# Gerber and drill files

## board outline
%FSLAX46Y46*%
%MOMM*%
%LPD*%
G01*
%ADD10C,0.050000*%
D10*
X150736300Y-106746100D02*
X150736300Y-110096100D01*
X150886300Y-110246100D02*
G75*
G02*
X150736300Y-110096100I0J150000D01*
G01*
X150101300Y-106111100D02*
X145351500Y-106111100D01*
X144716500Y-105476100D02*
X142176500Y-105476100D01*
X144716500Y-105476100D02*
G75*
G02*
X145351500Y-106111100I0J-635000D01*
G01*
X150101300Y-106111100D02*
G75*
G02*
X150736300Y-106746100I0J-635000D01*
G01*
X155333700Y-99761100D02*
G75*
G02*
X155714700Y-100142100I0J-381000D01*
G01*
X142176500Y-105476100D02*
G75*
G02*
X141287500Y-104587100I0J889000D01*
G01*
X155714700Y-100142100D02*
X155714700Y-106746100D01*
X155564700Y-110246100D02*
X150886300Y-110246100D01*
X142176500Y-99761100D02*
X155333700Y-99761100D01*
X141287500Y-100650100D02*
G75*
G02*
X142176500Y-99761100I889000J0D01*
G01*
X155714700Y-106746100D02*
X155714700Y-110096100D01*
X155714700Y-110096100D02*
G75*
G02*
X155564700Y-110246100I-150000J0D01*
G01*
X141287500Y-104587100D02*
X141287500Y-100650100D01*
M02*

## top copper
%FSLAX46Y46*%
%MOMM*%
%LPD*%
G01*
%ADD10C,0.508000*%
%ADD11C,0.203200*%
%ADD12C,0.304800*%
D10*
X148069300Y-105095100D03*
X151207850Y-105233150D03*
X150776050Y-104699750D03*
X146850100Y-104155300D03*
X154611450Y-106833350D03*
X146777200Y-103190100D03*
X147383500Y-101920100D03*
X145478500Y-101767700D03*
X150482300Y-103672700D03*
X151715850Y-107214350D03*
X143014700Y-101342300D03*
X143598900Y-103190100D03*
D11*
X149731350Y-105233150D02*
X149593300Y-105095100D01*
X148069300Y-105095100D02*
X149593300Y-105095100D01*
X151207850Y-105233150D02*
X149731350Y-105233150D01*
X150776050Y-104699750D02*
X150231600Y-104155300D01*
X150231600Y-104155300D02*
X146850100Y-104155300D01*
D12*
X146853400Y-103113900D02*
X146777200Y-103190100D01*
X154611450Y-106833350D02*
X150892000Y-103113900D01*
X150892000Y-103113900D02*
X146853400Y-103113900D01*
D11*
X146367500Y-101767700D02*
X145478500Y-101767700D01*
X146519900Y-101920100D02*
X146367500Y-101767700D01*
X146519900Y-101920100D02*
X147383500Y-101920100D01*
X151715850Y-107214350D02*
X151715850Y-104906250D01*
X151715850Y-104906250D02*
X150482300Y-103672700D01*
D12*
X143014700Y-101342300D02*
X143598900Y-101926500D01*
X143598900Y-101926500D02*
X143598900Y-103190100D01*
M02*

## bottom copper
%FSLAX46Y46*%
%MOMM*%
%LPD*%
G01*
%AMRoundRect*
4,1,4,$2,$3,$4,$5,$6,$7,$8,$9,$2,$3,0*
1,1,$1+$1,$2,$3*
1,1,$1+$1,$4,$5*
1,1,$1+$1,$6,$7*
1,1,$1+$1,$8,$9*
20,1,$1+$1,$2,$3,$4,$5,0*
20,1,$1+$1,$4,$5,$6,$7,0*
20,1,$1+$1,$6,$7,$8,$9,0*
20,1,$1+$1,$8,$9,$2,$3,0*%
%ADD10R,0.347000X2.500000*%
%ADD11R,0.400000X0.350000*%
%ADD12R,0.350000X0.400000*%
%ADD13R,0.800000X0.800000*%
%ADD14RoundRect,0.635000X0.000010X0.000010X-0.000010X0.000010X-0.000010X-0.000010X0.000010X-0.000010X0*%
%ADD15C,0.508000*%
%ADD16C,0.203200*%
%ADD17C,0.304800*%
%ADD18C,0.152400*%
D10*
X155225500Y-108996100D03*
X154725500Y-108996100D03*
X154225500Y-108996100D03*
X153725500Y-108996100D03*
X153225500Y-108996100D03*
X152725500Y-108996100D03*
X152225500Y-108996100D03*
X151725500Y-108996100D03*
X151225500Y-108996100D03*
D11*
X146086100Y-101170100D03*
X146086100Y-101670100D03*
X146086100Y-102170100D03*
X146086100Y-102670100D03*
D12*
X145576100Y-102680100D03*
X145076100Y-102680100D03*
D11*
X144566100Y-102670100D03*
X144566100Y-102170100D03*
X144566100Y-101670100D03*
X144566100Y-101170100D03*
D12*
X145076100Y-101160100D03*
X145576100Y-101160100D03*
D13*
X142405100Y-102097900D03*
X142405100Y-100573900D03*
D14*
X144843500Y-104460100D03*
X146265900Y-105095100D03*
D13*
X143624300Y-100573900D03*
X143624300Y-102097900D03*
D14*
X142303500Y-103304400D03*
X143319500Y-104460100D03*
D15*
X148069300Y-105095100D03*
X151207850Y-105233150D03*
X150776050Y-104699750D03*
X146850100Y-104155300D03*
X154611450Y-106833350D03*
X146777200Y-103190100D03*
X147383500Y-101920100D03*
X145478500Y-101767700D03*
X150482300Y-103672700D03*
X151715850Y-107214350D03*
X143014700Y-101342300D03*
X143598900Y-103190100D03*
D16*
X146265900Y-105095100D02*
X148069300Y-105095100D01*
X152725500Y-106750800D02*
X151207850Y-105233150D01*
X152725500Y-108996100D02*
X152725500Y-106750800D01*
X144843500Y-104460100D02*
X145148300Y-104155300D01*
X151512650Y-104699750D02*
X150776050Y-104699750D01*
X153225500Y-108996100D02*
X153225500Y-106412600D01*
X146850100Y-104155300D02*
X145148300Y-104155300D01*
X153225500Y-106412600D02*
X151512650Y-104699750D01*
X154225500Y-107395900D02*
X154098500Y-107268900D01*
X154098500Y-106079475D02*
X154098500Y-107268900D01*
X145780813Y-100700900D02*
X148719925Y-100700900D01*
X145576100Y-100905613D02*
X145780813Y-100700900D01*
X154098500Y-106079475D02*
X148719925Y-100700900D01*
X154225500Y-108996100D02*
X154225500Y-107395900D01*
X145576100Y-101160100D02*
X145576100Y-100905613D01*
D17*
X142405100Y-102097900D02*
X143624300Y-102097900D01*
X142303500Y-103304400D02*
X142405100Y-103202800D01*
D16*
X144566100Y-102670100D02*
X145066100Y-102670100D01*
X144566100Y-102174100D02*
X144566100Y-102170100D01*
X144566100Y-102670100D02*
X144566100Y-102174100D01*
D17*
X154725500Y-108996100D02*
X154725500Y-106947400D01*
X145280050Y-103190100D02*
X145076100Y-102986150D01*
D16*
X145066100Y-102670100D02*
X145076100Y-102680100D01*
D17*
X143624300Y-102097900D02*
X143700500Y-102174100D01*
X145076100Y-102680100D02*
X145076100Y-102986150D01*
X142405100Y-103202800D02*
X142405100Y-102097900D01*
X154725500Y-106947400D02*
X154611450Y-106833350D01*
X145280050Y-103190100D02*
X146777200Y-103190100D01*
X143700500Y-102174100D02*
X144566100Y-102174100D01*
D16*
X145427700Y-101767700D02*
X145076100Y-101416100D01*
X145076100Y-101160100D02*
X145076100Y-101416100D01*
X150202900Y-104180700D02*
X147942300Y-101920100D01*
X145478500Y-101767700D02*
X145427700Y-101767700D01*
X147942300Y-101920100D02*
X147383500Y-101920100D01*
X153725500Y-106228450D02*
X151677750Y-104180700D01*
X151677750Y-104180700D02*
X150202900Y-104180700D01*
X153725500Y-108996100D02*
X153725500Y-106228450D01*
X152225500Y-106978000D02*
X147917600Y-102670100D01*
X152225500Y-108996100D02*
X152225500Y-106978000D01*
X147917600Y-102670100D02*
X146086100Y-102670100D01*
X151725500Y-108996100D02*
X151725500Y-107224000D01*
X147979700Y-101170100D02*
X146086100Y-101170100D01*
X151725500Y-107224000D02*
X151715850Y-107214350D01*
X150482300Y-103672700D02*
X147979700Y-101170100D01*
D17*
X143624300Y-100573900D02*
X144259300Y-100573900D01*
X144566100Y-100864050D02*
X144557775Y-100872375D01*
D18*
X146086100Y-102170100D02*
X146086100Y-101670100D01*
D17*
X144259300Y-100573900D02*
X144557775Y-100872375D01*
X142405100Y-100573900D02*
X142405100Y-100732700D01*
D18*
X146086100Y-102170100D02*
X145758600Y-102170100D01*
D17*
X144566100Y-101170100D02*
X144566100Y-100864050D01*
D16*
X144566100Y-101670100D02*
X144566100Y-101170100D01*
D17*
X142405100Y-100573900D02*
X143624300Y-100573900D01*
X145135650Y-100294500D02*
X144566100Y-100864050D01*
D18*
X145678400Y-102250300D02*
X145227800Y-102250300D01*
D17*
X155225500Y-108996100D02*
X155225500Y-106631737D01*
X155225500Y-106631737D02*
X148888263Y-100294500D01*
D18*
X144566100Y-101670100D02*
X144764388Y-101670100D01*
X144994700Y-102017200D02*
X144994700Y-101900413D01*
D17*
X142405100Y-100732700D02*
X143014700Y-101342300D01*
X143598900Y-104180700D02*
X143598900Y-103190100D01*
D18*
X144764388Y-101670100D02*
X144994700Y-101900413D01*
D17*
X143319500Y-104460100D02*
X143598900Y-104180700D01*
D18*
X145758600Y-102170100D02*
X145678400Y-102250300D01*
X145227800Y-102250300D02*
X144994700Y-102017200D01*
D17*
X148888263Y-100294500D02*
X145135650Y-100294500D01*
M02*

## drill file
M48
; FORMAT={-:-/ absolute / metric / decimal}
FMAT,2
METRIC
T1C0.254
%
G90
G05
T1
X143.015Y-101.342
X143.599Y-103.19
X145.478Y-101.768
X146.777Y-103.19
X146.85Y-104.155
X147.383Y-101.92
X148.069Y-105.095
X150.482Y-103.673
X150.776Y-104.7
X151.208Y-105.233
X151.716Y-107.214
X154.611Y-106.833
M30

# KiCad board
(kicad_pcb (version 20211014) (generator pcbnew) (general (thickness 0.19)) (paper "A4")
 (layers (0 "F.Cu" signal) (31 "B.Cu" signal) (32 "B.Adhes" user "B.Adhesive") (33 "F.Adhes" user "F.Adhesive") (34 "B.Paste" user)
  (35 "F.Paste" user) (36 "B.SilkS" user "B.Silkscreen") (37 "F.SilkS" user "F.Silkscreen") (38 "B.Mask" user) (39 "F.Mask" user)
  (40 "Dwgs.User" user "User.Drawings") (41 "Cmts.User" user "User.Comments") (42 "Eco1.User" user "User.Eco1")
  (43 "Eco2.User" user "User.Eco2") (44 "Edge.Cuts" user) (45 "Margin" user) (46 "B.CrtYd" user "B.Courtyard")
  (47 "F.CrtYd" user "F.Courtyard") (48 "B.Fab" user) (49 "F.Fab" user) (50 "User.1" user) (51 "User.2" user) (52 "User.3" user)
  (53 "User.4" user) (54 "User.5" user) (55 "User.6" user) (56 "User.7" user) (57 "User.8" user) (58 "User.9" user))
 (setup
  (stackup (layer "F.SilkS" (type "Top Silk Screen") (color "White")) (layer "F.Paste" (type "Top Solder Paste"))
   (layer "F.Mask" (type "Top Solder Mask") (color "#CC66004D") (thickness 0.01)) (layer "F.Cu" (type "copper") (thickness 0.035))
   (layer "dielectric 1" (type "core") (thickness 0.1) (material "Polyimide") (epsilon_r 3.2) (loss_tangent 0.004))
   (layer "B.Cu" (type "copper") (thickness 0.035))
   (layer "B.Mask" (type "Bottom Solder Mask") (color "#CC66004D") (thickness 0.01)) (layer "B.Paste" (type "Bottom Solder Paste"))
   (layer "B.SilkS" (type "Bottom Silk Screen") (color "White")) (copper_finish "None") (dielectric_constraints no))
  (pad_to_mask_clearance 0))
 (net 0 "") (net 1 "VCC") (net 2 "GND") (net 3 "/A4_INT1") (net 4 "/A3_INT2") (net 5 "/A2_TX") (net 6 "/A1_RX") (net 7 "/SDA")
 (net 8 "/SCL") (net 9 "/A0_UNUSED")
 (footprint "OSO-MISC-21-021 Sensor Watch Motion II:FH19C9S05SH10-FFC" (layer "F.Cu") (at 153.2255 106.7461)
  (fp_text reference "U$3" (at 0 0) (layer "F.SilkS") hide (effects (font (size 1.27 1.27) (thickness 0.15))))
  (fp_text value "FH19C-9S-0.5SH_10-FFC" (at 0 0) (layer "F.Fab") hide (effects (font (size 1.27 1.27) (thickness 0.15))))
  (pad "1" smd rect (at 2 2.25 90) (size 2.5 0.347) (layers "B.Cu" "B.Mask") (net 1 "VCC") (solder_mask_margin 0.0635))
  (pad "2" smd rect (at 1.5 2.25 90) (size 2.5 0.347) (layers "B.Cu" "B.Mask") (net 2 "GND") (solder_mask_margin 0.0635))
  (pad "3" smd rect (at 1 2.25 90) (size 2.5 0.347) (layers "B.Cu" "B.Mask") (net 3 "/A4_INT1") (solder_mask_margin 0.0635))
  (pad "4" smd rect (at 0.5 2.25 90) (size 2.5 0.347) (layers "B.Cu" "B.Mask") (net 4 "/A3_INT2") (solder_mask_margin 0.0635))
  (pad "5" smd rect (at 0 2.25 90) (size 2.5 0.347) (layers "B.Cu" "B.Mask") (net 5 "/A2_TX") (solder_mask_margin 0.0635))
  (pad "6" smd rect (at -0.5 2.25 90) (size 2.5 0.347) (layers "B.Cu" "B.Mask") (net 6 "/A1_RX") (solder_mask_margin 0.0635))
  (pad "7" smd rect (at -1 2.25 90) (size 2.5 0.347) (layers "B.Cu" "B.Mask") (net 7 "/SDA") (solder_mask_margin 0.0635))
  (pad "8" smd rect (at -1.5 2.25 90) (size 2.5 0.347) (layers "B.Cu" "B.Mask") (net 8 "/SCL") (solder_mask_margin 0.0635))
  (pad "9" smd rect (at -2 2.25 90) (size 2.5 0.347) (layers "B.Cu" "B.Mask") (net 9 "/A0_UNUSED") (solder_mask_margin 0.0635)))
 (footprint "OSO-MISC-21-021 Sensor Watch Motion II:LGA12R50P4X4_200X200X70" (layer "B.Cu") (at 145.3261 101.9201 180)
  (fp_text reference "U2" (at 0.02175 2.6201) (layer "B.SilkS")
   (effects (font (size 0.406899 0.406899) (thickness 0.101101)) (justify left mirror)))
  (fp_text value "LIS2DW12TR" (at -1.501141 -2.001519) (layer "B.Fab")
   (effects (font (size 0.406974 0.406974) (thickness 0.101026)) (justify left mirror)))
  (pad "1" smd rect (at -0.76 0.75 180) (size 0.4 0.35) (layers "B.Cu" "B.Paste" "B.Mask") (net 8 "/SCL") (solder_mask_margin 0.0635))
  (pad "2" smd rect (at -0.76 0.25 180) (size 0.4 0.35) (layers "B.Cu" "B.Paste" "B.Mask") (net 1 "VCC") (solder_mask_margin 0.0635))
  (pad "3" smd rect (at -0.76 -0.25 180) (size 0.4 0.35) (layers "B.Cu" "B.Paste" "B.Mask") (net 1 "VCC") (solder_mask_margin 0.0635))
  (pad "4" smd rect (at -0.76 -0.75 180) (size 0.4 0.35) (layers "B.Cu" "B.Paste" "B.Mask") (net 7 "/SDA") (solder_mask_margin 0.0635))
  (pad "5" smd rect (at -0.25 -0.76 180) (size 0.35 0.4) (layers "B.Cu" "B.Paste" "B.Mask") (solder_mask_margin 0.0635))
  (pad "6" smd rect (at 0.25 -0.76 180) (size 0.35 0.4) (layers "B.Cu" "B.Paste" "B.Mask") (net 2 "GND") (solder_mask_margin 0.0635))
  (pad "7" smd rect (at 0.76 -0.75 180) (size 0.4 0.35) (layers "B.Cu" "B.Paste" "B.Mask") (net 2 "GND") (solder_mask_margin 0.0635))
  (pad "8" smd rect (at 0.76 -0.25 180) (size 0.4 0.35) (layers "B.Cu" "B.Paste" "B.Mask") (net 2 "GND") (solder_mask_margin 0.0635))
  (pad "9" smd rect (at 0.76 0.25 180) (size 0.4 0.35) (layers "B.Cu" "B.Paste" "B.Mask") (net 1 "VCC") (solder_mask_margin 0.0635))
  (pad "10" smd rect (at 0.76 0.75 180) (size 0.4 0.35) (layers "B.Cu" "B.Paste" "B.Mask") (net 1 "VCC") (solder_mask_margin 0.0635))
  (pad "11" smd rect (at 0.25 0.76 180) (size 0.35 0.4) (layers "B.Cu" "B.Paste" "B.Mask") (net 4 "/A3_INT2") (solder_mask_margin 0.0635))
  (pad "12" smd rect (at -0.25 0.76 180) (size 0.35 0.4) (layers "B.Cu" "B.Paste" "B.Mask") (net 3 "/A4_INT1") (solder_mask_margin 0.0635)))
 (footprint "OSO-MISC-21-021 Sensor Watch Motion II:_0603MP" (layer "B.Cu") (at 142.4051 101.3359 90)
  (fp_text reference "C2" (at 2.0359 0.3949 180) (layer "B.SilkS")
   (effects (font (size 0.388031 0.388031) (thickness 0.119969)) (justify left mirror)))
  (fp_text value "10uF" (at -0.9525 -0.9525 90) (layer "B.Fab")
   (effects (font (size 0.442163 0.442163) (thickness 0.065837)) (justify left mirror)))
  (pad "1" smd rect (at -0.762 0 90) (size 0.8 0.8) (layers "B.Cu" "B.Paste" "B.Mask") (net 2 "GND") (solder_mask_margin 0.0635))
  (pad "2" smd rect (at 0.762 0 90) (size 0.8 0.8) (layers "B.Cu" "B.Paste" "B.Mask") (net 1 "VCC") (solder_mask_margin 0.0635)))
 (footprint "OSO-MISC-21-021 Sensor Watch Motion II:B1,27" (layer "B.Cu") (at 144.8435 104.4601 180)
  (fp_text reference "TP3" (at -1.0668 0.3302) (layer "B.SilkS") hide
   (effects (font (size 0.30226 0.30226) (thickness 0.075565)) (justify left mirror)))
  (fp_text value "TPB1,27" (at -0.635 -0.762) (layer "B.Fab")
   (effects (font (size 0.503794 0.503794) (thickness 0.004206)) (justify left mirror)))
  (pad "TP" smd roundrect (at 0 0 180) (size 1.27 1.27) (layers "B.Cu" "B.Mask") (roundrect_rratio 0.5) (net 5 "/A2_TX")
   (solder_mask_margin 0.0635)))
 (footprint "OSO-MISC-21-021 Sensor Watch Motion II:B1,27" (layer "B.Cu") (at 146.2659 105.0951 180)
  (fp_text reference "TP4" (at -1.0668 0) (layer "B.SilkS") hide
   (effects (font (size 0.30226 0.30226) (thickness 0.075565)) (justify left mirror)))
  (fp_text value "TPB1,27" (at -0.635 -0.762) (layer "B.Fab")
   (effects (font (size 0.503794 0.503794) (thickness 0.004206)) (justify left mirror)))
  (pad "TP" smd roundrect (at 0 0 180) (size 1.27 1.27) (layers "B.Cu" "B.Mask") (roundrect_rratio 0.5) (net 6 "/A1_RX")
   (solder_mask_margin 0.0635)))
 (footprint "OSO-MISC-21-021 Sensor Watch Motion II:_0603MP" (layer "B.Cu") (at 143.6243 101.3359 -90)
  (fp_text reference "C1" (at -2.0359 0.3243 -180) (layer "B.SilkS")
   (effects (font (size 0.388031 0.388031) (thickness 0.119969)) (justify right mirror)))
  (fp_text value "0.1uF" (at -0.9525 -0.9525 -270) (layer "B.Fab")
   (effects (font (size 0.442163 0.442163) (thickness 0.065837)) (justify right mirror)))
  (pad "1" smd rect (at -0.762 0 270) (size 0.8 0.8) (layers "B.Cu" "B.Paste" "B.Mask") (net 1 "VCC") (solder_mask_margin 0.0635))
  (pad "2" smd rect (at 0.762 0 270) (size 0.8 0.8) (layers "B.Cu" "B.Paste" "B.Mask") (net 2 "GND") (solder_mask_margin 0.0635)))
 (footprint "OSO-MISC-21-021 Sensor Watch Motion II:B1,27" (layer "B.Cu") (at 142.3035 103.3044 180)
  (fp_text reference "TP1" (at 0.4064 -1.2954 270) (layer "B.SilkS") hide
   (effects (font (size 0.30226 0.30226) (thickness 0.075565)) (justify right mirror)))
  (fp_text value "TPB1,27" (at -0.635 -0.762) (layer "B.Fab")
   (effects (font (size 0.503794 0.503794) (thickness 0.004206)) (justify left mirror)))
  (pad "TP" smd roundrect (at 0 0 180) (size 1.27 1.27) (layers "B.Cu" "B.Mask") (roundrect_rratio 0.5) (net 2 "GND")
   (solder_mask_margin 0.0635)))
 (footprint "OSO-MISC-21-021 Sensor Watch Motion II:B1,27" (layer "B.Cu") (at 143.3195 104.4601 180)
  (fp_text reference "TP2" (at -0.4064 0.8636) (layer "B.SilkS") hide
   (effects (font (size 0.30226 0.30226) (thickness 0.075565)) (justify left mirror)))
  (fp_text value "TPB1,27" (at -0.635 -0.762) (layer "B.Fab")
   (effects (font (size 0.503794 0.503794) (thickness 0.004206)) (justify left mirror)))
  (pad "TP" smd roundrect (at 0 0 180) (size 1.27 1.27) (layers "B.Cu" "B.Mask") (roundrect_rratio 0.5) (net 1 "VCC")
   (solder_mask_margin 0.0635)))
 (gr_line (start 150.7363 106.7461) (end 150.7363 110.0961) (layer "Edge.Cuts") (width 0.05))
 (gr_arc (start 150.8863 110.2461) (mid 150.780234 110.202166) (end 150.7363 110.0961) (layer "Edge.Cuts") (width 0.05))
 (gr_line (start 150.1013 106.1111) (end 145.3515 106.1111) (layer "Edge.Cuts") (width 0.05))
 (gr_line (start 144.7165 105.4761) (end 142.1765 105.4761) (layer "Edge.Cuts") (width 0.05))
 (gr_arc (start 144.7165 105.4761) (mid 145.165513 105.662087) (end 145.3515 106.1111) (layer "Edge.Cuts") (width 0.05))
 (gr_arc (start 150.1013 106.1111) (mid 150.550313 106.297087) (end 150.7363 106.7461) (layer "Edge.Cuts") (width 0.05))
 (gr_arc (start 155.3337 99.7611) (mid 155.603108 99.872692) (end 155.7147 100.1421) (layer "Edge.Cuts") (width 0.05))
 (gr_arc (start 142.1765 105.4761) (mid 141.547882 105.215718) (end 141.2875 104.5871) (layer "Edge.Cuts") (width 0.05))
 (gr_line (start 155.7147 100.1421) (end 155.7147 106.7461) (layer "Edge.Cuts") (width 0.05))
 (gr_line (start 155.5647 110.2461) (end 150.8863 110.2461) (layer "Edge.Cuts") (width 0.05))
 (gr_line (start 142.1765 99.7611) (end 155.3337 99.7611) (layer "Edge.Cuts") (width 0.05))
 (gr_arc (start 141.2875 100.6501) (mid 141.547882 100.021482) (end 142.1765 99.7611) (layer "Edge.Cuts") (width 0.05))
 (gr_line (start 155.7147 106.7461) (end 155.7147 110.0961) (layer "Edge.Cuts") (width 0.05))
 (gr_arc (start 155.7147 110.0961) (mid 155.670766 110.202166) (end 155.5647 110.2461) (layer "Edge.Cuts") (width 0.05))
 (gr_line (start 141.2875 104.5871) (end 141.2875 100.6501) (layer "Edge.Cuts") (width 0.05))
 (segment (start 149.73135 105.23315) (end 149.5933 105.0951) (width 0.2032) (layer "F.Cu") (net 6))
 (segment (start 148.0693 105.0951) (end 149.5933 105.0951) (width 0.2032) (layer "F.Cu") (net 6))
 (segment (start 151.20785 105.23315) (end 149.73135 105.23315) (width 0.2032) (layer "F.Cu") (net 6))
 (via (at 148.0693 105.0951) (size 0.508) (drill 0.254) (layers "F.Cu" "B.Cu") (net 6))
 (via (at 151.20785 105.23315) (size 0.508) (drill 0.254) (layers "F.Cu" "B.Cu") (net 6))
 (segment (start 146.2659 105.0951) (end 148.0693 105.0951) (width 0.2032) (layer "B.Cu") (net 6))
 (segment (start 152.7255 106.7508) (end 151.20785 105.23315) (width 0.2032) (layer "B.Cu") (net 6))
 (segment (start 152.7255 108.9961) (end 152.7255 106.7508) (width 0.2032) (layer "B.Cu") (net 6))
 (segment (start 150.77605 104.69975) (end 150.2316 104.1553) (width 0.2032) (layer "F.Cu") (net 5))
 (segment (start 150.2316 104.1553) (end 146.8501 104.1553) (width 0.2032) (layer "F.Cu") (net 5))
 (via (at 150.77605 104.69975) (size 0.508) (drill 0.254) (layers "F.Cu" "B.Cu") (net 5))
 (via (at 146.8501 104.1553) (size 0.508) (drill 0.254) (layers "F.Cu" "B.Cu") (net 5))
 (segment (start 144.8435 104.4601) (end 145.1483 104.1553) (width 0.2032) (layer "B.Cu") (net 5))
 (segment (start 151.51265 104.69975) (end 150.77605 104.69975) (width 0.2032) (layer "B.Cu") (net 5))
 (segment (start 153.2255 108.9961) (end 153.2255 106.4126) (width 0.2032) (layer "B.Cu") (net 5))
 (segment (start 146.8501 104.1553) (end 145.1483 104.1553) (width 0.2032) (layer "B.Cu") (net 5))
 (segment (start 153.2255 106.4126) (end 151.51265 104.69975) (width 0.2032) (layer "B.Cu") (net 5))
 (segment (start 154.2255 107.3959) (end 154.0985 107.2689) (width 0.2032) (layer "B.Cu") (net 3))
 (segment (start 154.0985 106.079475) (end 154.0985 107.2689) (width 0.2032) (layer "B.Cu") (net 3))
 (segment (start 145.780813 100.7009) (end 148.719925 100.7009) (width 0.2032) (layer "B.Cu") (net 3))
 (segment (start 145.5761 100.905613) (end 145.780813 100.7009) (width 0.2032) (layer "B.Cu") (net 3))
 (segment (start 154.0985 106.079475) (end 148.719925 100.7009) (width 0.2032) (layer "B.Cu") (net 3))
 (segment (start 154.2255 108.9961) (end 154.2255 107.3959) (width 0.2032) (layer "B.Cu") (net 3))
 (segment (start 145.5761 101.1601) (end 145.5761 100.905613) (width 0.2032) (layer "B.Cu") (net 3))
 (segment (start 146.8534 103.1139) (end 146.7772 103.1901) (width 0.3048) (layer "F.Cu") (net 2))
 (segment (start 154.61145 106.83335) (end 150.892 103.1139) (width 0.3048) (layer "F.Cu") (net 2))
 (segment (start 150.892 103.1139) (end 146.8534 103.1139) (width 0.3048) (layer "F.Cu") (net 2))
 (via (at 154.61145 106.83335) (size 0.508) (drill 0.254) (layers "F.Cu" "B.Cu") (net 2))
 (via (at 146.7772 103.1901) (size 0.508) (drill 0.254) (layers "F.Cu" "B.Cu") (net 2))
 (segment (start 142.4051 102.0979) (end 143.6243 102.0979) (width 0.3048) (layer "B.Cu") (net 2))
 (segment (start 142.3035 103.3044) (end 142.4051 103.2028) (width 0.3048) (layer "B.Cu") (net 2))
 (segment (start 144.5661 102.6701) (end 145.0661 102.6701) (width 0.2032) (layer "B.Cu") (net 2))
 (segment (start 144.5661 102.1741) (end 144.5661 102.1701) (width 0.2032) (layer "B.Cu") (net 2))
 (segment (start 144.5661 102.6701) (end 144.5661 102.1741) (width 0.2032) (layer "B.Cu") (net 2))
 (segment (start 154.7255 108.9961) (end 154.7255 106.9474) (width 0.3048) (layer "B.Cu") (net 2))
 (segment (start 145.28005 103.1901) (end 145.0761 102.98615) (width 0.3048) (layer "B.Cu") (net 2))
 (segment (start 145.0661 102.6701) (end 145.0761 102.6801) (width 0.2032) (layer "B.Cu") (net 2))
 (segment (start 143.6243 102.0979) (end 143.7005 102.1741) (width 0.3048) (layer "B.Cu") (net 2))
 (segment (start 145.0761 102.6801) (end 145.0761 102.98615) (width 0.3048) (layer "B.Cu") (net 2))
 (segment (start 142.4051 103.2028) (end 142.4051 102.0979) (width 0.3048) (layer "B.Cu") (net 2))
 (segment (start 154.7255 106.9474) (end 154.61145 106.83335) (width 0.3048) (layer "B.Cu") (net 2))
 (segment (start 145.28005 103.1901) (end 146.7772 103.1901) (width 0.3048) (layer "B.Cu") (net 2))
 (segment (start 143.7005 102.1741) (end 144.5661 102.1741) (width 0.3048) (layer "B.Cu") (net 2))
 (segment (start 146.3675 101.7677) (end 145.4785 101.7677) (width 0.2032) (layer "F.Cu") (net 4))
 (segment (start 146.5199 101.9201) (end 146.3675 101.7677) (width 0.2032) (layer "F.Cu") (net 4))
 (segment (start 146.5199 101.9201) (end 147.3835 101.9201) (width 0.2032) (layer "F.Cu") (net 4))
 (via (at 147.3835 101.9201) (size 0.508) (drill 0.254) (layers "F.Cu" "B.Cu") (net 4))
 (via (at 145.4785 101.7677) (size 0.508) (drill 0.254) (layers "F.Cu" "B.Cu") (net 4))
 (segment (start 145.4277 101.7677) (end 145.0761 101.4161) (width 0.2032) (layer "B.Cu") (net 4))
 (segment (start 145.0761 101.1601) (end 145.0761 101.4161) (width 0.2032) (layer "B.Cu") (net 4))
 (segment (start 150.2029 104.1807) (end 147.9423 101.9201) (width 0.2032) (layer "B.Cu") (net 4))
 (segment (start 145.4785 101.7677) (end 145.4277 101.7677) (width 0.2032) (layer "B.Cu") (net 4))
 (segment (start 147.9423 101.9201) (end 147.3835 101.9201) (width 0.2032) (layer "B.Cu") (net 4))
 (segment (start 153.7255 106.22845) (end 151.67775 104.1807) (width 0.2032) (layer "B.Cu") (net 4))
 (segment (start 151.67775 104.1807) (end 150.2029 104.1807) (width 0.2032) (layer "B.Cu") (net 4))
 (segment (start 153.7255 108.9961) (end 153.7255 106.22845) (width 0.2032) (layer "B.Cu") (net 4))
 (segment (start 152.2255 106.978) (end 147.9176 102.6701) (width 0.2032) (layer "B.Cu") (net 7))
 (segment (start 152.2255 108.9961) (end 152.2255 106.978) (width 0.2032) (layer "B.Cu") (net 7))
 (segment (start 147.9176 102.6701) (end 146.0861 102.6701) (width 0.2032) (layer "B.Cu") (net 7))
 (segment (start 151.71585 107.21435) (end 151.71585 104.90625) (width 0.2032) (layer "F.Cu") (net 8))
 (segment (start 151.71585 104.90625) (end 150.4823 103.6727) (width 0.2032) (layer "F.Cu") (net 8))
 (via (at 150.4823 103.6727) (size 0.508) (drill 0.254) (layers "F.Cu" "B.Cu") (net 8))
 (via (at 151.71585 107.21435) (size 0.508) (drill 0.254) (layers "F.Cu" "B.Cu") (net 8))
 (segment (start 151.7255 108.9961) (end 151.7255 107.224) (width 0.2032) (layer "B.Cu") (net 8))
 (segment (start 147.9797 101.1701) (end 146.0861 101.1701) (width 0.2032) (layer "B.Cu") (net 8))
 (segment (start 151.7255 107.224) (end 151.71585 107.21435) (width 0.2032) (layer "B.Cu") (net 8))
 (segment (start 150.4823 103.6727) (end 147.9797 101.1701) (width 0.2032) (layer "B.Cu") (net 8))
 (segment (start 143.0147 101.3423) (end 143.5989 101.9265) (width 0.3048) (layer "F.Cu") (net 1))
 (segment (start 143.5989 101.9265) (end 143.5989 103.1901) (width 0.3048) (layer "F.Cu") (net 1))
 (via (at 143.0147 101.3423) (size 0.508) (drill 0.254) (layers "F.Cu" "B.Cu") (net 1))
 (via (at 143.5989 103.1901) (size 0.508) (drill 0.254) (layers "F.Cu" "B.Cu") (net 1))
 (segment (start 143.6243 100.5739) (end 144.2593 100.5739) (width 0.3048) (layer "B.Cu") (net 1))
 (segment (start 144.5661 100.86405) (end 144.557775 100.872375) (width 0.3048) (layer "B.Cu") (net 1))
 (segment (start 146.0861 102.1701) (end 146.0861 101.6701) (width 0.1524) (layer "B.Cu") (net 1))
 (segment (start 144.2593 100.5739) (end 144.557775 100.872375) (width 0.3048) (layer "B.Cu") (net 1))
 (segment (start 142.4051 100.5739) (end 142.4051 100.7327) (width 0.3048) (layer "B.Cu") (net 1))
 (segment (start 146.0861 102.1701) (end 145.7586 102.1701) (width 0.1524) (layer "B.Cu") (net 1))
 (segment (start 144.5661 101.1701) (end 144.5661 100.86405) (width 0.3048) (layer "B.Cu") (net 1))
 (segment (start 144.5661 101.6701) (end 144.5661 101.1701) (width 0.2032) (layer "B.Cu") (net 1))
 (segment (start 142.4051 100.5739) (end 143.6243 100.5739) (width 0.3048) (layer "B.Cu") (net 1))
 (segment (start 145.13565 100.2945) (end 144.5661 100.86405) (width 0.3048) (layer "B.Cu") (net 1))
 (segment (start 145.6784 102.2503) (end 145.2278 102.2503) (width 0.1524) (layer "B.Cu") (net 1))
 (segment (start 155.2255 108.9961) (end 155.2255 106.631737) (width 0.3048) (layer "B.Cu") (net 1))
 (segment (start 155.2255 106.631737) (end 148.888263 100.2945) (width 0.3048) (layer "B.Cu") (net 1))
 (segment (start 144.5661 101.6701) (end 144.764388 101.6701) (width 0.1524) (layer "B.Cu") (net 1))
 (segment (start 144.9947 102.0172) (end 144.9947 101.900413) (width 0.1524) (layer "B.Cu") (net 1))
 (segment (start 142.4051 100.7327) (end 143.0147 101.3423) (width 0.3048) (layer "B.Cu") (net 1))
 (segment (start 143.5989 104.1807) (end 143.5989 103.1901) (width 0.3048) (layer "B.Cu") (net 1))
 (segment (start 144.764388 101.6701) (end 144.9947 101.900413) (width 0.1524) (layer "B.Cu") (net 1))
 (segment (start 143.3195 104.4601) (end 143.5989 104.1807) (width 0.3048) (layer "B.Cu") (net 1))
 (segment (start 145.7586 102.1701) (end 145.6784 102.2503) (width 0.1524) (layer "B.Cu") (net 1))
 (segment (start 145.2278 102.2503) (end 144.9947 102.0172) (width 0.1524) (layer "B.Cu") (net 1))
 (segment (start 148.888263 100.2945) (end 145.13565 100.2945) (width 0.3048) (layer "B.Cu") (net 1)))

